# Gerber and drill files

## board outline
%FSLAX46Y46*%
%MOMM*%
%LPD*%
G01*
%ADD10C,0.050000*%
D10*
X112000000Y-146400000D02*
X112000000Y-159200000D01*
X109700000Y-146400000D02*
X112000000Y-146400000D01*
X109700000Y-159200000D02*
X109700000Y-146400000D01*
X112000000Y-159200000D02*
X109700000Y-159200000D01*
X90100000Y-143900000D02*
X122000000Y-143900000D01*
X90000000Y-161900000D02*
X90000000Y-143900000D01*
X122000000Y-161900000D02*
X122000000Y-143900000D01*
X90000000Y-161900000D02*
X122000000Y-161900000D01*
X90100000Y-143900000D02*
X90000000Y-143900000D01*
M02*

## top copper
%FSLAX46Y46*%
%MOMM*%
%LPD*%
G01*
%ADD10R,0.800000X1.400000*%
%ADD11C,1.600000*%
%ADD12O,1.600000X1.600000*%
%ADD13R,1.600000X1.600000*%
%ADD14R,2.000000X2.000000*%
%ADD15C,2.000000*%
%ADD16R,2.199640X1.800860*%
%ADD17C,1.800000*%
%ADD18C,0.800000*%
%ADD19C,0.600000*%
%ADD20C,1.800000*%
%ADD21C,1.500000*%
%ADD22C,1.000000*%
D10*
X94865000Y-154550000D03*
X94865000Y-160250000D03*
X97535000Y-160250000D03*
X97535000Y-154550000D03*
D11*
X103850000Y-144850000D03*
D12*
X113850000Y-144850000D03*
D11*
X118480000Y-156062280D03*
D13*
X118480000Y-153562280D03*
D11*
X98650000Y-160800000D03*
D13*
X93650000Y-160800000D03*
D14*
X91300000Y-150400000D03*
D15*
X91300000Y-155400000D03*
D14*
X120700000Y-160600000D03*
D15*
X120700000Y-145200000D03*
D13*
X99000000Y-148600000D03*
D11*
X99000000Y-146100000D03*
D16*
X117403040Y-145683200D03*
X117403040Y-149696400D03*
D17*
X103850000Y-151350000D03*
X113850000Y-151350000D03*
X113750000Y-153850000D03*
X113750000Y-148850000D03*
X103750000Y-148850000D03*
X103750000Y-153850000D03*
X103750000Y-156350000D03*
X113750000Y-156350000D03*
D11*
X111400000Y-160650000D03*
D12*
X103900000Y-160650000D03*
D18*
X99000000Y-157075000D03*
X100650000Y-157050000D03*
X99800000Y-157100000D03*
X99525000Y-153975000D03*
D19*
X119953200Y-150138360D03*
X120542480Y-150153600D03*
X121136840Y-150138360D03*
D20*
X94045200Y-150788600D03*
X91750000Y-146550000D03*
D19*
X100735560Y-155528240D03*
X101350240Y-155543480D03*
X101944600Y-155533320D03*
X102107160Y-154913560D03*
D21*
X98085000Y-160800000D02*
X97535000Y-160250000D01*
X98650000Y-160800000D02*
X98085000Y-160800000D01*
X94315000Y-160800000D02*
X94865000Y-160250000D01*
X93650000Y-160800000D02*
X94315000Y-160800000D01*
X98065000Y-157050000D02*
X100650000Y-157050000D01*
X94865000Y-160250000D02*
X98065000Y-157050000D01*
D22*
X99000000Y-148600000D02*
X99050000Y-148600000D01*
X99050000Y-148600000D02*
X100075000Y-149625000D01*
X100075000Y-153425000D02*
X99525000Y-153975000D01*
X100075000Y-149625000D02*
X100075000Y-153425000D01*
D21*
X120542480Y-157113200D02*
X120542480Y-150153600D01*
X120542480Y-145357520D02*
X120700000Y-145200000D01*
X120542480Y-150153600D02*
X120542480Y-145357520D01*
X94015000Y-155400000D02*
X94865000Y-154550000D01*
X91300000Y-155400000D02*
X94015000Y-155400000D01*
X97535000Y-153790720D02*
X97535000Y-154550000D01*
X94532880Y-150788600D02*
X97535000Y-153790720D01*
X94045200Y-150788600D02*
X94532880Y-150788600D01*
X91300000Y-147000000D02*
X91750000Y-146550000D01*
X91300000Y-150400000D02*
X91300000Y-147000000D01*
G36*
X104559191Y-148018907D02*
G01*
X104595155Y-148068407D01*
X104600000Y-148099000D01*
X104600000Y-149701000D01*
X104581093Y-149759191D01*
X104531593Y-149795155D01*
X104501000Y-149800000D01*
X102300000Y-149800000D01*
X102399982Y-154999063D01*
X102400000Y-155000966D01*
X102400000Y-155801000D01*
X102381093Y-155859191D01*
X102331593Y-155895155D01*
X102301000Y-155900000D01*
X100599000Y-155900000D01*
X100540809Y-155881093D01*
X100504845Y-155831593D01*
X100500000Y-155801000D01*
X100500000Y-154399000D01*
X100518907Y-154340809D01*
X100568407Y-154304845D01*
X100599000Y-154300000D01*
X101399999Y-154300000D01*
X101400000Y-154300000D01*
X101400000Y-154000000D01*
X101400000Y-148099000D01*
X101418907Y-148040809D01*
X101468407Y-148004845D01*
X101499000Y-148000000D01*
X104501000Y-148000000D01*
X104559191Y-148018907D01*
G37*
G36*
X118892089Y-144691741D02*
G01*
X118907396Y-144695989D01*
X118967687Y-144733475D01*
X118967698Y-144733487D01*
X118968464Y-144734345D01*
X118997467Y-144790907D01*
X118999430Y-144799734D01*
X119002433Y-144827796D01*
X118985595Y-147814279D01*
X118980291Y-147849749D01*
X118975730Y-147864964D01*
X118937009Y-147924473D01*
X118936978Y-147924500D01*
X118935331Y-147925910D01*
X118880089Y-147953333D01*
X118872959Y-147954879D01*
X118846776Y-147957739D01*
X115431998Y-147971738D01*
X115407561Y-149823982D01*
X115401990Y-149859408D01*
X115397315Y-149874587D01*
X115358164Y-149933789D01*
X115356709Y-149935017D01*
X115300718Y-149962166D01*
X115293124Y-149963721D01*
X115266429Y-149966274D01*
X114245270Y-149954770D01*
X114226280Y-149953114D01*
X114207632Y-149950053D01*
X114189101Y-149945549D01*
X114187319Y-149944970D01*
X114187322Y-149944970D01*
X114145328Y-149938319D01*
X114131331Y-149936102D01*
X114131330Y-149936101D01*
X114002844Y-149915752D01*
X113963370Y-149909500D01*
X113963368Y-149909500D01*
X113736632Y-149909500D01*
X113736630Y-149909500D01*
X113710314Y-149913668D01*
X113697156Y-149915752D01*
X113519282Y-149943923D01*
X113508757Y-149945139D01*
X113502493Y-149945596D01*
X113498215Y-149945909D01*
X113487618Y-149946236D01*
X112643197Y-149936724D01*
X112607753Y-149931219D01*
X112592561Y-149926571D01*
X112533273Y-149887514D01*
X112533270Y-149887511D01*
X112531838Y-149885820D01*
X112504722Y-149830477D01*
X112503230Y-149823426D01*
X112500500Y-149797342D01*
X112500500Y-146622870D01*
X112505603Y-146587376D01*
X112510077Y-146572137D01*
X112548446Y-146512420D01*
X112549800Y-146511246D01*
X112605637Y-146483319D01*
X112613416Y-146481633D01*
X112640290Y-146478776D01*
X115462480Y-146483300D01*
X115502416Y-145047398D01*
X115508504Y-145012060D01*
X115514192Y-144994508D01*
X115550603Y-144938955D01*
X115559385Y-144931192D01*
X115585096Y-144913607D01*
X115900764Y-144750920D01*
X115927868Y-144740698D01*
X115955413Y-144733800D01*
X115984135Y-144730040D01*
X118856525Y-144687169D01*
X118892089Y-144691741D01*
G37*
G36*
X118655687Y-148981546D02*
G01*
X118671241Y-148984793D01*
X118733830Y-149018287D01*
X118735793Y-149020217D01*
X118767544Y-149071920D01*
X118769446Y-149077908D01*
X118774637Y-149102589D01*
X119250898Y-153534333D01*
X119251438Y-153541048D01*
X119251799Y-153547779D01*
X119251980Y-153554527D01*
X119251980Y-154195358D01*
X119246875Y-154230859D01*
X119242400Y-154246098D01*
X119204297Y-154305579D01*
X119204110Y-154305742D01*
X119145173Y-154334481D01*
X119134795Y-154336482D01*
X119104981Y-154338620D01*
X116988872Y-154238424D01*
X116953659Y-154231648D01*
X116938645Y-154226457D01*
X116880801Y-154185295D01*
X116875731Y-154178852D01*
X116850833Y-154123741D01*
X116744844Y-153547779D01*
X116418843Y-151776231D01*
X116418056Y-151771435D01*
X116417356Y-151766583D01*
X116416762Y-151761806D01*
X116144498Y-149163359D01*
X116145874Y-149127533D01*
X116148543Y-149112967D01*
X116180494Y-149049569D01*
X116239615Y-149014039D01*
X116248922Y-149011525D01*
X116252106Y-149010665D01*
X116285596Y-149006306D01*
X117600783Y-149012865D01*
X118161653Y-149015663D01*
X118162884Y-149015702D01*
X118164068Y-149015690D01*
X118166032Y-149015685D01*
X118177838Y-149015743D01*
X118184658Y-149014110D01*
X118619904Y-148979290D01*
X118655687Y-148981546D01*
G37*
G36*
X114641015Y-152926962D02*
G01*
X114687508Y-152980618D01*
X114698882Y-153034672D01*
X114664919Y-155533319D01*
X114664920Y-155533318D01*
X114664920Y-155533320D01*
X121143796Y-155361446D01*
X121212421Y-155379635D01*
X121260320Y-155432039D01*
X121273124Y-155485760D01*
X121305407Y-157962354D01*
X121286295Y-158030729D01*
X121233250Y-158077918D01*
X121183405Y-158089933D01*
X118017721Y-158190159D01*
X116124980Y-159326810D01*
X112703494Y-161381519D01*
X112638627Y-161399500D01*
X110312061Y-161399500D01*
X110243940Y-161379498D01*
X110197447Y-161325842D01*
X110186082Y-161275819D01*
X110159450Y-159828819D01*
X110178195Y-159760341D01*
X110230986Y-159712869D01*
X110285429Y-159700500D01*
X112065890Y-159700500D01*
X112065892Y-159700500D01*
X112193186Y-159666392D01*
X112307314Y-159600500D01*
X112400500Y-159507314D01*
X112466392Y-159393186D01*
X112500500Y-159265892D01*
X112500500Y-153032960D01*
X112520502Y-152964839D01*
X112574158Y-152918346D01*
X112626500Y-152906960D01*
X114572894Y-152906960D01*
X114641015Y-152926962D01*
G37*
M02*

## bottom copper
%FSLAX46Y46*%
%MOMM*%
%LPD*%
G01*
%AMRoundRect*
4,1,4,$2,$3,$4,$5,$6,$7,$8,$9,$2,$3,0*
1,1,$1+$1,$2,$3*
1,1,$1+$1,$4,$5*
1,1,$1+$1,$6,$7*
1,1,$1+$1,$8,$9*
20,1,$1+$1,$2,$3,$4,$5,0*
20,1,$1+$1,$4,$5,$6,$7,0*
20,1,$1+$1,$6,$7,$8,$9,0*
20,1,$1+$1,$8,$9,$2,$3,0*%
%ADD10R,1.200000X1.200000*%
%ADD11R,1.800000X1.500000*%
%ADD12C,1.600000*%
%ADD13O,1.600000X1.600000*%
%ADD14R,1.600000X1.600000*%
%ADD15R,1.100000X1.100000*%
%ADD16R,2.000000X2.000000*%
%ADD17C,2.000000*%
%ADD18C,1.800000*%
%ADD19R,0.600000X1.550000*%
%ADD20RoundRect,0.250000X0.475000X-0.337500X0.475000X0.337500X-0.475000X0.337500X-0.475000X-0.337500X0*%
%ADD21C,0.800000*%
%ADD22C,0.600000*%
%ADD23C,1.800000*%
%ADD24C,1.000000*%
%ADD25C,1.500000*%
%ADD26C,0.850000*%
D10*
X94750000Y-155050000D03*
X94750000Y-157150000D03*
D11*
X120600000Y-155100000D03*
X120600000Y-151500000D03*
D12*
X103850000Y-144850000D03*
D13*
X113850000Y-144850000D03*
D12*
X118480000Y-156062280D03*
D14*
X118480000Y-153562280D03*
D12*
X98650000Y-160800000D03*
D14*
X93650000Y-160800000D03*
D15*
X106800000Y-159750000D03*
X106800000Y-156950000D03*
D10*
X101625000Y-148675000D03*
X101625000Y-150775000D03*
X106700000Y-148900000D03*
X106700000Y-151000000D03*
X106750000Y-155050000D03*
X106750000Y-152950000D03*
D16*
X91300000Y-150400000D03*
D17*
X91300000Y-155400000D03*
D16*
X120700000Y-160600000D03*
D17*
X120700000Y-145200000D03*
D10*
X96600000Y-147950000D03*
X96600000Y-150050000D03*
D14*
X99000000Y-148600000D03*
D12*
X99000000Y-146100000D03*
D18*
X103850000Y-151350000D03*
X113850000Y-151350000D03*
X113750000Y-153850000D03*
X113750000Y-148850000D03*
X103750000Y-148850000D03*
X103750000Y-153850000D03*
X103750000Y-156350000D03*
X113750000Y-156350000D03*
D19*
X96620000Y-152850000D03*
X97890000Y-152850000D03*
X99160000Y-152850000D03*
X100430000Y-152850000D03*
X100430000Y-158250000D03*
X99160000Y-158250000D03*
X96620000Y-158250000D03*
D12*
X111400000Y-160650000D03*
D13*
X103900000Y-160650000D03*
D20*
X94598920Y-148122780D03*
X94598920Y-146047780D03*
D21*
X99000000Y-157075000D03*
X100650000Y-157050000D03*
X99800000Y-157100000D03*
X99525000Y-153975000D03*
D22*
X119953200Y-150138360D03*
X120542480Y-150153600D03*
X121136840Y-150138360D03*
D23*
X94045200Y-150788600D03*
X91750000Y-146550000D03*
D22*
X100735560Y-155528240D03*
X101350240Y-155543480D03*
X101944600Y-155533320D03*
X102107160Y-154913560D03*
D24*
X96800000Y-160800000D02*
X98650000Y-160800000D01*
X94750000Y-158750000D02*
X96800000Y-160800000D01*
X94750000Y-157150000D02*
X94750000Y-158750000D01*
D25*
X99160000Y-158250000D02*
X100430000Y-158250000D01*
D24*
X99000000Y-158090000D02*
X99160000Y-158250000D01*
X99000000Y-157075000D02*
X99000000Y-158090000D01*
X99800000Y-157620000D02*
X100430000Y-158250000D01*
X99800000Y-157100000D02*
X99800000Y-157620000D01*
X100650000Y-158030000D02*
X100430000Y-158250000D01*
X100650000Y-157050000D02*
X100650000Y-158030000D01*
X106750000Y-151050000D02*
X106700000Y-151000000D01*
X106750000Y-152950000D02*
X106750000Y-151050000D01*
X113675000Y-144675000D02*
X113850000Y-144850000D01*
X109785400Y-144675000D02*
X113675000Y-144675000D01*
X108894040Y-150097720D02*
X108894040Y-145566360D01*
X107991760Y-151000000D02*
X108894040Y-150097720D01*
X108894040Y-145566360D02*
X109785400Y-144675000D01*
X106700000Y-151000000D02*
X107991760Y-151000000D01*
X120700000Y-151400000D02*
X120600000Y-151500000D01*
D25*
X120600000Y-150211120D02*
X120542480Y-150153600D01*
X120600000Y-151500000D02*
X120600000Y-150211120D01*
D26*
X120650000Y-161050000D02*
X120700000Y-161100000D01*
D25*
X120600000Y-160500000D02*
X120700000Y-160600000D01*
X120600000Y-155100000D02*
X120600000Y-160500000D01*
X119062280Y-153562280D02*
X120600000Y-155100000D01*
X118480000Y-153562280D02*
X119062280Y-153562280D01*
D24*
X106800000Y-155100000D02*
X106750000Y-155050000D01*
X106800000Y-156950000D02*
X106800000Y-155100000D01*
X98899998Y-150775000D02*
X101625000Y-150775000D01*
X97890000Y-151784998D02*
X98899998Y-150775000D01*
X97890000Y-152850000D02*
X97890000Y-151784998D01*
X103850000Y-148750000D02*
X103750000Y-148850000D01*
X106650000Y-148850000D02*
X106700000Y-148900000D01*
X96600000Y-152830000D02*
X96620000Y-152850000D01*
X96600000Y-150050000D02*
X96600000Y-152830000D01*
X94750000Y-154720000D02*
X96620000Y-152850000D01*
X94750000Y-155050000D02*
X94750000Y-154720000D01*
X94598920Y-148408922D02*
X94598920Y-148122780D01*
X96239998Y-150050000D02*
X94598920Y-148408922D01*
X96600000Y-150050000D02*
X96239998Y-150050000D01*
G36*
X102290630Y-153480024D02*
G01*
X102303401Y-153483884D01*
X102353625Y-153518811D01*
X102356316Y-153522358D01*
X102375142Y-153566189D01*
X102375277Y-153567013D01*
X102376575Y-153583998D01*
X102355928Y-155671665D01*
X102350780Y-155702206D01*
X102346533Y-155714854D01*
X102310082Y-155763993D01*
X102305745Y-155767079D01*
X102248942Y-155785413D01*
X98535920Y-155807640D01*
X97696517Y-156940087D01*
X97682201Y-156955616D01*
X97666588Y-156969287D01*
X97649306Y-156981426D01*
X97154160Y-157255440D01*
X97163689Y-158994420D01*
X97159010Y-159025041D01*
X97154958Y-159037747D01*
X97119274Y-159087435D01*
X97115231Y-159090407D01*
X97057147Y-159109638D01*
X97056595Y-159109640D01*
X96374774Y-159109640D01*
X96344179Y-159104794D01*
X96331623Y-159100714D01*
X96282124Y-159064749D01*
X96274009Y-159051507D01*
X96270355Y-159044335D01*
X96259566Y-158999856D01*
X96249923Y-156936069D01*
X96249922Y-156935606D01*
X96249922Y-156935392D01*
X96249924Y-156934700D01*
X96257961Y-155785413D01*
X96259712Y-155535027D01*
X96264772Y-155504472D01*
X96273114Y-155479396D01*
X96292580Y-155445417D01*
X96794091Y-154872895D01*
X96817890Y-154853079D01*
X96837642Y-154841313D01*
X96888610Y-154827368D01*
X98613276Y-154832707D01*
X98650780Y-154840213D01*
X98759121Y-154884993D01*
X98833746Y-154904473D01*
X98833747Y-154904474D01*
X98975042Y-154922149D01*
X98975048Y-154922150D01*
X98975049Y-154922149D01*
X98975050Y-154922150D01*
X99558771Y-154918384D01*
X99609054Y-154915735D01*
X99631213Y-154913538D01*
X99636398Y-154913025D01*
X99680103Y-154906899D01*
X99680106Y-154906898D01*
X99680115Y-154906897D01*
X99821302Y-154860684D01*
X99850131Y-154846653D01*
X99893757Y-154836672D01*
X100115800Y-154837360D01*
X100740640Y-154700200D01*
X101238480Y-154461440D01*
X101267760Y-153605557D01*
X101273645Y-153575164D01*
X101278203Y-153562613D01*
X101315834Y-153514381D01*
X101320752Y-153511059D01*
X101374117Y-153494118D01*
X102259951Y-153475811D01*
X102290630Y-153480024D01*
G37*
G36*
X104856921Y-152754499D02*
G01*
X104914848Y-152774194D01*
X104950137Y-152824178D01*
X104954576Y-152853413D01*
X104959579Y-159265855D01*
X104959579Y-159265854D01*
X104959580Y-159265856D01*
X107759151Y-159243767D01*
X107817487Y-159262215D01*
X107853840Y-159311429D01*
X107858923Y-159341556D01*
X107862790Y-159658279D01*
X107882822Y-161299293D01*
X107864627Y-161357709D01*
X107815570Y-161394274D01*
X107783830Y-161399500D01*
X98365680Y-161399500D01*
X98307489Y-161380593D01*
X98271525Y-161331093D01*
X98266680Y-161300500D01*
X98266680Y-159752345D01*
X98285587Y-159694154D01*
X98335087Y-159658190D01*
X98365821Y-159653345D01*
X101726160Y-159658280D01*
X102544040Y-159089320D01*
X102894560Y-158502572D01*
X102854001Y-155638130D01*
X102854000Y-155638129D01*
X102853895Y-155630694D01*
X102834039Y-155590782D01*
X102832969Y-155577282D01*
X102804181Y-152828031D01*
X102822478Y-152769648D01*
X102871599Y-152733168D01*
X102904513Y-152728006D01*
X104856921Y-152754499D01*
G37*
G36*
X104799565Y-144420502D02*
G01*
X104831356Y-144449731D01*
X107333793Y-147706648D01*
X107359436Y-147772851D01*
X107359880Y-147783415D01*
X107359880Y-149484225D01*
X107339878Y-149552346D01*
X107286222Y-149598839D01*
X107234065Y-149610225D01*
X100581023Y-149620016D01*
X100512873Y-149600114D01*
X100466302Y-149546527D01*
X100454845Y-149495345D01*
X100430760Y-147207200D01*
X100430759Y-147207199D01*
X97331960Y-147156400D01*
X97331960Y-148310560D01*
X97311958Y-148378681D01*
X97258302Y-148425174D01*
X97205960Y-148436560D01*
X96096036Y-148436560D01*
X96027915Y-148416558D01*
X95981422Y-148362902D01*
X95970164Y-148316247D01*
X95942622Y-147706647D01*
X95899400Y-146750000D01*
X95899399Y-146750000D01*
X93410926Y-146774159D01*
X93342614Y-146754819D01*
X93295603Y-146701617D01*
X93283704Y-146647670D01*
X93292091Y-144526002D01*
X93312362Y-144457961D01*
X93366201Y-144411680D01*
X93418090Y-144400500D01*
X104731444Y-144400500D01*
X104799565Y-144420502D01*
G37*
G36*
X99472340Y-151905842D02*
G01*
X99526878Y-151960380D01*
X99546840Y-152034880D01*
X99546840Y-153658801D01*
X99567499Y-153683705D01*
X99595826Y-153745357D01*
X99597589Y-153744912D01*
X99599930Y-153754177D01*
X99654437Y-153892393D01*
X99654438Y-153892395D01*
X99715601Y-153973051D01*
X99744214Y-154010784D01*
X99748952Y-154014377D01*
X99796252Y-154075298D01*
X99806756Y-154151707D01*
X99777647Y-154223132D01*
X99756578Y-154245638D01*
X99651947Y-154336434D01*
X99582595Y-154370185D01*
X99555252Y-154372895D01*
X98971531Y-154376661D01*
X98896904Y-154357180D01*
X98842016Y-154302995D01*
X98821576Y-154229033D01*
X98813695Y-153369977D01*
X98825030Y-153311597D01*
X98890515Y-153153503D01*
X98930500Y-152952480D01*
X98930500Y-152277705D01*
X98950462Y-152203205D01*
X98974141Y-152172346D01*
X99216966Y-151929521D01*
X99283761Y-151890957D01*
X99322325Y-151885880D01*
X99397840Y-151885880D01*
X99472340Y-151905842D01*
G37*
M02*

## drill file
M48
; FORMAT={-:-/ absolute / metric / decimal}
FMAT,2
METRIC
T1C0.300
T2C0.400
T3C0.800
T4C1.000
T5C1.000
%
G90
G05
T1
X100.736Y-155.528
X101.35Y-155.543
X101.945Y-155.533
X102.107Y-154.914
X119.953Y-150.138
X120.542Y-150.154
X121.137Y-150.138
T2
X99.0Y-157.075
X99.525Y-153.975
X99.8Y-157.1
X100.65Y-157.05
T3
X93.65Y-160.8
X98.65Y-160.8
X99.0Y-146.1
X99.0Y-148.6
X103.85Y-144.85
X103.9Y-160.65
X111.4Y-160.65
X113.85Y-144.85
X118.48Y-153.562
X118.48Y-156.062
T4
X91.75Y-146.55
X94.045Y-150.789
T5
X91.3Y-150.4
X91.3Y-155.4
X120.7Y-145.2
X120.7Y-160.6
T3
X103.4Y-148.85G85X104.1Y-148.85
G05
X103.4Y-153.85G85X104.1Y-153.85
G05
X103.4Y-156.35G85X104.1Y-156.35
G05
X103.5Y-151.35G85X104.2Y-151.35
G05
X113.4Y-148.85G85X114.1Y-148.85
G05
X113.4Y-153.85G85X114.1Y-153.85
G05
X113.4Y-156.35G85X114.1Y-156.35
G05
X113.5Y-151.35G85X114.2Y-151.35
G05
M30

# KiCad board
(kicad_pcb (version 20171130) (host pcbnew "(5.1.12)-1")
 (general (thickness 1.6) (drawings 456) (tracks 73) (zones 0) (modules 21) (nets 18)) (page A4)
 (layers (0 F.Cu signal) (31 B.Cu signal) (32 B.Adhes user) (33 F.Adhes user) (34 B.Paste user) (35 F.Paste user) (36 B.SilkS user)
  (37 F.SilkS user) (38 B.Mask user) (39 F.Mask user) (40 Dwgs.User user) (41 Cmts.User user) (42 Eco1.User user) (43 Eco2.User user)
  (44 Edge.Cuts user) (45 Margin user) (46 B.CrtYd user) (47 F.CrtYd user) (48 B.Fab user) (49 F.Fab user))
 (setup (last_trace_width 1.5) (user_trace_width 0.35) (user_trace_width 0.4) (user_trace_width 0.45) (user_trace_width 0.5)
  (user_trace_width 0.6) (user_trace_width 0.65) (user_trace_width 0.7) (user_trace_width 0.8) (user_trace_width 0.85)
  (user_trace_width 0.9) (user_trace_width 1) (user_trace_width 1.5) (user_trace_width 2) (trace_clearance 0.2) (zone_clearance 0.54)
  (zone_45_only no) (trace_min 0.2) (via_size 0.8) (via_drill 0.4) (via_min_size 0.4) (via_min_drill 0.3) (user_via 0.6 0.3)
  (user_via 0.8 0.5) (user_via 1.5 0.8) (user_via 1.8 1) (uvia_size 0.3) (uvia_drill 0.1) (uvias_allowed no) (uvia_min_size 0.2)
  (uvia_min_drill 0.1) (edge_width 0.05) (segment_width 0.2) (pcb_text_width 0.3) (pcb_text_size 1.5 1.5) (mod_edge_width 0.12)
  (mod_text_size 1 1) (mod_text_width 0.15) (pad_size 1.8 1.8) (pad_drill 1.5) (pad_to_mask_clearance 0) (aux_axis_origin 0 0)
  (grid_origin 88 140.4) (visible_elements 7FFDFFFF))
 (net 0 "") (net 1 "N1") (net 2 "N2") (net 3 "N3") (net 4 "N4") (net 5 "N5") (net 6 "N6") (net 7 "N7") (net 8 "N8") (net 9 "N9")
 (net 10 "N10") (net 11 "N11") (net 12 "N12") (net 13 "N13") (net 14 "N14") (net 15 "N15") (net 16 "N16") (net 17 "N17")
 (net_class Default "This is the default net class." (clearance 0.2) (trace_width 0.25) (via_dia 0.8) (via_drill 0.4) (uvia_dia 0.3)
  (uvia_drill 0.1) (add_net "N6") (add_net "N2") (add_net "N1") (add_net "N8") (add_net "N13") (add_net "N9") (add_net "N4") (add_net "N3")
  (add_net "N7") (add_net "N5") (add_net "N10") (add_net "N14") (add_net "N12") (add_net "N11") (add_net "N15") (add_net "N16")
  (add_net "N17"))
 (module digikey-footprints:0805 (layer B.Cu) (at 94.75 156.1 90)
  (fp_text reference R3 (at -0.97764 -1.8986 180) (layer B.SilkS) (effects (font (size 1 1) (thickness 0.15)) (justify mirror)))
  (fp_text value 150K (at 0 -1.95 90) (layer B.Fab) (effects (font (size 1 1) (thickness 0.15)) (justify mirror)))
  (pad 2 smd rect (at 1.05 0 90) (size 1.2 1.2) (layers B.Cu B.Paste B.Mask) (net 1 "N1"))
  (pad 1 smd rect (at -1.05 0 90) (size 1.2 1.2) (layers B.Cu B.Paste B.Mask) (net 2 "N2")))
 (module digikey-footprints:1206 (layer B.Cu) (at 120.6 153.3 90)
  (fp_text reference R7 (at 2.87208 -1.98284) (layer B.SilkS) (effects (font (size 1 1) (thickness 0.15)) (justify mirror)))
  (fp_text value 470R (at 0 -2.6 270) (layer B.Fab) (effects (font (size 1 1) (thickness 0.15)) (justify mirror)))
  (pad 1 smd rect (at -1.8 0 90) (size 1.5 1.8) (layers B.Cu B.Paste B.Mask) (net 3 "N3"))
  (pad 2 smd rect (at 1.8 0 90) (size 1.5 1.8) (layers B.Cu B.Paste B.Mask) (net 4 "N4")))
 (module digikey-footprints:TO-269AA (layer F.Cu) (at 96.2 157.4)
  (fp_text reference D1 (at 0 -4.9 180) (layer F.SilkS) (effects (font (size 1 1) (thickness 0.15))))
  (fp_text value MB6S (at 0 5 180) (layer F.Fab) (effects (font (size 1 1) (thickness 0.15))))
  (pad 4 smd rect (at -1.335 -2.85) (size 0.8 1.4) (layers F.Cu F.Paste F.Mask) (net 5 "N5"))
  (pad 1 smd rect (at -1.335 2.85) (size 0.8 1.4) (layers F.Cu F.Paste F.Mask) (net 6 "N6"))
  (pad 2 smd rect (at 1.335 2.85) (size 0.8 1.4) (layers F.Cu F.Paste F.Mask) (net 2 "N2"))
  (pad 3 smd rect (at 1.335 -2.85) (size 0.8 1.4) (layers F.Cu F.Paste F.Mask) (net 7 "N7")))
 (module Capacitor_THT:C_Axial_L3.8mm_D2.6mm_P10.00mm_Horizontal (layer B.Cu) (at 103.85 144.85)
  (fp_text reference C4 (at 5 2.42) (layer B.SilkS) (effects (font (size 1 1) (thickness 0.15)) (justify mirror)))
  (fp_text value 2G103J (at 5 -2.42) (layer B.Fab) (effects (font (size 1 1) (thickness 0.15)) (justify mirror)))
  (pad 1 thru_hole circle (at 0 0) (size 1.6 1.6) (drill 0.8) (layers *.Cu *.Mask) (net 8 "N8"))
  (pad 2 thru_hole oval (at 10 0) (size 1.6 1.6) (drill 0.8) (layers *.Cu *.Mask) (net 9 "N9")))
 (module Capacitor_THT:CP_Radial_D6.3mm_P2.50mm (layer B.Cu) (at 118.48 153.56228 270)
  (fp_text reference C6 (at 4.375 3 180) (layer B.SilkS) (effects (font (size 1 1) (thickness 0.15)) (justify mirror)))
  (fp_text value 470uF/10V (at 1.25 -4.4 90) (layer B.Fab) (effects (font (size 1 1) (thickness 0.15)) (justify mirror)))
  (pad 2 thru_hole circle (at 2.5 0 270) (size 1.6 1.6) (drill 0.8) (layers *.Cu *.Mask) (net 4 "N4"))
  (pad 1 thru_hole rect (at 0 0 270) (size 1.6 1.6) (drill 0.8) (layers *.Cu *.Mask) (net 3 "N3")))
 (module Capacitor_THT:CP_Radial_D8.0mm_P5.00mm (layer B.Cu) (at 93.65 160.8)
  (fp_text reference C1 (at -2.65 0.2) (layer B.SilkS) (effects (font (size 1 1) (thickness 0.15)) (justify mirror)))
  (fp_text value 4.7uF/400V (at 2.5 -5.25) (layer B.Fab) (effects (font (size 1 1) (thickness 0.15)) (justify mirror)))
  (pad 2 thru_hole circle (at 5 0) (size 1.6 1.6) (drill 0.8) (layers *.Cu *.Mask) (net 2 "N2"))
  (pad 1 thru_hole rect (at 0 0) (size 1.6 1.6) (drill 0.8) (layers *.Cu *.Mask) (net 6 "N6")))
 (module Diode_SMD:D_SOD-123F (layer B.Cu) (at 106.8 158.35 90)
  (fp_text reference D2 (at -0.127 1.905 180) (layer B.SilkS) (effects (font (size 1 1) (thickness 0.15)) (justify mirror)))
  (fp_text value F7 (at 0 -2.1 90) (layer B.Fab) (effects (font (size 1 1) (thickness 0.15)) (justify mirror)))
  (pad 1 smd rect (at -1.4 0 90) (size 1.1 1.1) (layers B.Cu B.Paste B.Mask) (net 2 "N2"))
  (pad 2 smd rect (at 1.4 0 90) (size 1.1 1.1) (layers B.Cu B.Paste B.Mask) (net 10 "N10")))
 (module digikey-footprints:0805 (layer B.Cu) (at 101.625 149.725 270)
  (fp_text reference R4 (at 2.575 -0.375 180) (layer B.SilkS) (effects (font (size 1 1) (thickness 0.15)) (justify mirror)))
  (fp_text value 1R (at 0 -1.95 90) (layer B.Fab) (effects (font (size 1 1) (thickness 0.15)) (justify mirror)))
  (pad 1 smd rect (at -1.05 0 270) (size 1.2 1.2) (layers B.Cu B.Paste B.Mask) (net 8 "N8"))
  (pad 2 smd rect (at 1.05 0 270) (size 1.2 1.2) (layers B.Cu B.Paste B.Mask) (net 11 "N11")))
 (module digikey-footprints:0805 (layer B.Cu) (at 106.7 149.95 90)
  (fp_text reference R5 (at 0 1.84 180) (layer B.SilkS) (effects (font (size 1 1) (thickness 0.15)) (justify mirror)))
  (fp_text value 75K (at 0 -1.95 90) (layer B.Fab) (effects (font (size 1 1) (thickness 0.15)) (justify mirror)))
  (pad 2 smd rect (at 1.05 0 90) (size 1.2 1.2) (layers B.Cu B.Paste B.Mask) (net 8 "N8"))
  (pad 1 smd rect (at -1.05 0 90) (size 1.2 1.2) (layers B.Cu B.Paste B.Mask) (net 9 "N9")))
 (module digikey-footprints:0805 (layer B.Cu) (at 106.75 154 90)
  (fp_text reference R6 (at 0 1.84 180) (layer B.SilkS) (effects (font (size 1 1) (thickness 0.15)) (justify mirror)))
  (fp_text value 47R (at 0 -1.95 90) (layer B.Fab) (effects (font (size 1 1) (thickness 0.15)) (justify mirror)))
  (pad 1 smd rect (at -1.05 0 90) (size 1.2 1.2) (layers B.Cu B.Paste B.Mask) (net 10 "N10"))
  (pad 2 smd rect (at 1.05 0 90) (size 1.2 1.2) (layers B.Cu B.Paste B.Mask) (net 9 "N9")))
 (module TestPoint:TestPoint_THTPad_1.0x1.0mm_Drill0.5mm (layer F.Cu) (at 91.3 150.4)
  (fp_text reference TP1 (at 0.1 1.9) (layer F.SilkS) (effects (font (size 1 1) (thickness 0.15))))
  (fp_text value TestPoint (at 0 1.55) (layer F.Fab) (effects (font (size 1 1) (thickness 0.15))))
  (pad 1 thru_hole rect (at 0 0) (size 2 2) (drill 1) (layers *.Cu *.Mask) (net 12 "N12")))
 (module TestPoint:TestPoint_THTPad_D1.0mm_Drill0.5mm (layer F.Cu) (at 91.3 155.4)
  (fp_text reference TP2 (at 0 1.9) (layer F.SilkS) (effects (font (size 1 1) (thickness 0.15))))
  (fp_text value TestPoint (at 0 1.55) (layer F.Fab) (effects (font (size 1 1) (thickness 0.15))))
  (pad 1 thru_hole circle (at 0 0) (size 2 2) (drill 1) (layers *.Cu *.Mask) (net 5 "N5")))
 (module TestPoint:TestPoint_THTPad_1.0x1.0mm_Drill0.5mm (layer F.Cu) (at 120.7 160.6)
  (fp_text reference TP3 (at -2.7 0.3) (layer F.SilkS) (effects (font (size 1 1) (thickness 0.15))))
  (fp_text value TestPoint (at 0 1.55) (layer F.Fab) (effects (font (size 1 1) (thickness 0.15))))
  (pad 1 thru_hole rect (at 0 0) (size 2 2) (drill 1) (layers *.Cu *.Mask) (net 3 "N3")))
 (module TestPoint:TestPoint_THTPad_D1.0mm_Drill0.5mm (layer F.Cu) (at 120.7 145.2)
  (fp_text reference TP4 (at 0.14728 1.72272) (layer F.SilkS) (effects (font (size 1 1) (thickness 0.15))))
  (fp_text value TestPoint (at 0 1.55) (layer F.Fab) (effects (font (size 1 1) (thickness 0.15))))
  (pad 1 thru_hole circle (at 0 0) (size 2 2) (drill 1) (layers *.Cu *.Mask) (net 4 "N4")))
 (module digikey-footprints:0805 (layer B.Cu) (at 96.6 149 90)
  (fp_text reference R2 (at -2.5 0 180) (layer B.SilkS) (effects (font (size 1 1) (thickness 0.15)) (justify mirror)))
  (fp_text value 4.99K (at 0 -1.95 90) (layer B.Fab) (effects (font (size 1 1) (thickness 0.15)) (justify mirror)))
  (pad 2 smd rect (at 1.05 0 90) (size 1.2 1.2) (layers B.Cu B.Paste B.Mask) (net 8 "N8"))
  (pad 1 smd rect (at -1.05 0 90) (size 1.2 1.2) (layers B.Cu B.Paste B.Mask) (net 1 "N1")))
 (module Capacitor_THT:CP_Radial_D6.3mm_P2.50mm (layer F.Cu) (at 99 148.6 90)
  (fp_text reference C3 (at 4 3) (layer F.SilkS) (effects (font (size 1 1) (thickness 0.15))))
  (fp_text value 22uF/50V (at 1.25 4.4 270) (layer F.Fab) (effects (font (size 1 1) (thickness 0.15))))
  (pad 1 thru_hole rect (at 0 0 90) (size 1.6 1.6) (drill 0.8) (layers *.Cu *.Mask) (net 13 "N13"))
  (pad 2 thru_hole circle (at 2.5 0 90) (size 1.6 1.6) (drill 0.8) (layers *.Cu *.Mask) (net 8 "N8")))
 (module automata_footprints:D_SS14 (layer F.Cu) (at 117.40304 147.6898 90)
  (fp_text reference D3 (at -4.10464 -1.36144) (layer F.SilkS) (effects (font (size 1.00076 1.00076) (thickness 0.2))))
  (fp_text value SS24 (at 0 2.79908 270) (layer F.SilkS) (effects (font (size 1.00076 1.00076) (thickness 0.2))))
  (pad 2 smd rect (at 2.0066 0 90) (size 1.80086 2.19964) (layers F.Cu F.Paste F.Mask) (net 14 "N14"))
  (pad 1 smd rect (at -2.0066 0 90) (size 1.80086 2.19964) (layers F.Cu F.Paste F.Mask) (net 3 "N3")))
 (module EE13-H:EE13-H (layer F.Cu) (at 108.75 151.35)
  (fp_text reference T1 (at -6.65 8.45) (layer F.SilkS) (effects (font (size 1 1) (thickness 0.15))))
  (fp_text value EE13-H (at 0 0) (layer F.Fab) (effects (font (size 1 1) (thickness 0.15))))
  (pad 2 thru_hole circle (at -4.9 0) (size 1.8 1.8) (drill oval 1.5 0.8) (layers *.Cu *.Mask) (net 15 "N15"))
  (pad 7 thru_hole circle (at 5.1 0) (size 1.8 1.8) (drill oval 1.5 0.8) (layers *.Cu *.Mask) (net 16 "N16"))
  (pad 6 thru_hole circle (at 5 2.5) (size 1.8 1.8) (drill oval 1.5 0.8) (layers *.Cu *.Mask) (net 4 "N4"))
  (pad 8 thru_hole circle (at 5 -2.5) (size 1.8 1.8) (drill oval 1.5 0.8) (layers *.Cu *.Mask) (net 14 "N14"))
  (pad 1 thru_hole circle (at -5 -2.5) (size 1.8 1.8) (drill oval 1.5 0.8) (layers *.Cu *.Mask) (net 8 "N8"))
  (pad 3 thru_hole circle (at -5 2.5) (size 1.8 1.8) (drill oval 1.5 0.8) (layers *.Cu *.Mask) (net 2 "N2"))
  (pad 4 thru_hole circle (at -5 5) (size 1.8 1.8) (drill oval 1.5 0.8) (layers *.Cu *.Mask) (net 2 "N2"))
  (pad 5 thru_hole circle (at 5 5) (size 1.8 1.8) (drill oval 1.5 0.8) (layers *.Cu *.Mask) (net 4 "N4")))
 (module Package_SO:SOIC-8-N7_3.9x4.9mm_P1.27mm (layer B.Cu) (at 98.525 155.55 270)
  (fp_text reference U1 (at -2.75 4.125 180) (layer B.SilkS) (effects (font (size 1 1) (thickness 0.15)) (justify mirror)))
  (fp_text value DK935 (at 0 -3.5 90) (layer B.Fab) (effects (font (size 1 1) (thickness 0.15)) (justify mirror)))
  (pad 1 smd rect (at -2.7 1.905 270) (size 1.55 0.6) (layers B.Cu B.Paste B.Mask) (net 1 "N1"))
  (pad 2 smd rect (at -2.7 0.635 270) (size 1.55 0.6) (layers B.Cu B.Paste B.Mask) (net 11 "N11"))
  (pad 3 smd rect (at -2.7 -0.635 270) (size 1.55 0.6) (layers B.Cu B.Paste B.Mask) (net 13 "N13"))
  (pad 4 smd rect (at -2.7 -1.905 270) (size 1.55 0.6) (layers B.Cu B.Paste B.Mask) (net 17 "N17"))
  (pad 5 smd rect (at 2.7 -1.905 270) (size 1.55 0.6) (layers B.Cu B.Paste B.Mask) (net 6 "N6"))
  (pad 6 smd rect (at 2.7 -0.635 270) (size 1.55 0.6) (layers B.Cu B.Paste B.Mask) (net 6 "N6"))
  (pad 8 smd rect (at 2.7 1.905 270) (size 1.55 0.6) (layers B.Cu B.Paste B.Mask) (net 8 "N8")))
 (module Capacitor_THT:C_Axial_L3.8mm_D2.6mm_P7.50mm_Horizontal (layer F.Cu) (at 111.4 160.65 180)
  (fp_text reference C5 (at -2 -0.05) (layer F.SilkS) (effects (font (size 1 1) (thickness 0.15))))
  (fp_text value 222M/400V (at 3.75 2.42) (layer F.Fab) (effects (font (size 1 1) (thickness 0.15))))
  (pad 1 thru_hole circle (at 0 0 180) (size 1.6 1.6) (drill 0.8) (layers *.Cu *.Mask) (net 4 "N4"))
  (pad 2 thru_hole oval (at 7.5 0 180) (size 1.6 1.6) (drill 0.8) (layers *.Cu *.Mask) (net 2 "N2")))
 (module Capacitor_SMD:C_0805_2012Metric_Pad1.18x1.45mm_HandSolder (layer B.Cu) (at 94.59892 147.08528 90)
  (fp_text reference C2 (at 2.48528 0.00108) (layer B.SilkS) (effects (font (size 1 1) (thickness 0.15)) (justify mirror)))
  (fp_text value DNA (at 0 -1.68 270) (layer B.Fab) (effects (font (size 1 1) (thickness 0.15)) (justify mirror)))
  (pad 1 smd roundrect (at -1.0375 0 90) (size 1.175 1.45) (layers B.Cu B.Paste B.Mask) (roundrect_rratio 0.212766) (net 1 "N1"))
  (pad 2 smd roundrect (at 1.0375 0 90) (size 1.175 1.45) (layers B.Cu B.Paste B.Mask) (roundrect_rratio 0.212766) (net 8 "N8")))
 (gr_line (start 112 146.4) (end 112 159.2) (layer Edge.Cuts) (width 0.05))
 (gr_line (start 109.7 146.4) (end 112 146.4) (layer Edge.Cuts) (width 0.05))
 (gr_line (start 109.7 159.2) (end 109.7 146.4) (layer Edge.Cuts) (width 0.05))
 (gr_line (start 112 159.2) (end 109.7 159.2) (layer Edge.Cuts) (width 0.05))
 (gr_line (start 90.1 143.9) (end 122 143.9) (layer Edge.Cuts) (width 0.05))
 (gr_line (start 90 161.9) (end 90 143.9) (layer Edge.Cuts) (width 0.05))
 (gr_line (start 122 161.9) (end 122 143.9) (layer Edge.Cuts) (width 0.05))
 (gr_line (start 90 161.9) (end 122 161.9) (layer Edge.Cuts) (width 0.05))
 (gr_line (start 90.1 143.9) (end 90 143.9) (layer Edge.Cuts) (width 0.05))
 (segment (start 98.085 160.8) (end 97.535 160.25) (width 1.5) (layer F.Cu) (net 2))
 (segment (start 98.65 160.8) (end 98.085 160.8) (width 1.5) (layer F.Cu) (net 2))
 (segment (start 96.8 160.8) (end 98.65 160.8) (width 1) (layer B.Cu) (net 2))
 (segment (start 94.75 158.75) (end 96.8 160.8) (width 1) (layer B.Cu) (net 2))
 (segment (start 94.75 157.15) (end 94.75 158.75) (width 1) (layer B.Cu) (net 2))
 (via (at 99 157.075) (size 0.8) (drill 0.4) (layers F.Cu B.Cu) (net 6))
 (via (at 100.65 157.05) (size 0.8) (drill 0.4) (layers F.Cu B.Cu) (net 6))
 (via (at 99.8 157.1) (size 0.8) (drill 0.4) (layers F.Cu B.Cu) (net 6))
 (segment (start 94.315 160.8) (end 94.865 160.25) (width 1.5) (layer F.Cu) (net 6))
 (segment (start 93.65 160.8) (end 94.315 160.8) (width 1.5) (layer F.Cu) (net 6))
 (segment (start 98.065 157.05) (end 100.65 157.05) (width 1.5) (layer F.Cu) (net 6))
 (segment (start 94.865 160.25) (end 98.065 157.05) (width 1.5) (layer F.Cu) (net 6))
 (segment (start 99.16 158.25) (end 100.43 158.25) (width 1.5) (layer B.Cu) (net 6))
 (segment (start 99 158.09) (end 99.16 158.25) (width 1) (layer B.Cu) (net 6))
 (segment (start 99 157.075) (end 99 158.09) (width 1) (layer B.Cu) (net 6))
 (segment (start 99.8 157.62) (end 100.43 158.25) (width 1) (layer B.Cu) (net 6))
 (segment (start 99.8 157.1) (end 99.8 157.62) (width 1) (layer B.Cu) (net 6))
 (segment (start 100.65 158.03) (end 100.43 158.25) (width 1) (layer B.Cu) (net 6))
 (segment (start 100.65 157.05) (end 100.65 158.03) (width 1) (layer B.Cu) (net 6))
 (segment (start 99 148.6) (end 99.05 148.6) (width 1) (layer F.Cu) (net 13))
 (segment (start 99.05 148.6) (end 100.075 149.625) (width 1) (layer F.Cu) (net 13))
 (segment (start 100.075 153.425) (end 99.525 153.975) (width 1) (layer F.Cu) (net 13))
 (segment (start 100.075 149.625) (end 100.075 153.425) (width 1) (layer F.Cu) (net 13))
 (via (at 99.525 153.975) (size 0.8) (drill 0.4) (layers F.Cu B.Cu) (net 13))
 (segment (start 106.75 151.05) (end 106.7 151) (width 1) (layer B.Cu) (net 9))
 (segment (start 106.75 152.95) (end 106.75 151.05) (width 1) (layer B.Cu) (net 9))
 (segment (start 113.675 144.675) (end 113.85 144.85) (width 1) (layer B.Cu) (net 9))
 (segment (start 109.7854 144.675) (end 113.675 144.675) (width 1) (layer B.Cu) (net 9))
 (segment (start 108.89404 150.09772) (end 108.89404 145.56636) (width 1) (layer B.Cu) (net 9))
 (segment (start 107.99176 151) (end 108.89404 150.09772) (width 1) (layer B.Cu) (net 9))
 (segment (start 108.89404 145.56636) (end 109.7854 144.675) (width 1) (layer B.Cu) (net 9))
 (segment (start 106.7 151) (end 107.99176 151) (width 1) (layer B.Cu) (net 9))
 (via (at 119.9532 150.13836) (size 0.6) (drill 0.3) (layers F.Cu B.Cu) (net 4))
 (via (at 120.54248 150.1536) (size 0.6) (drill 0.3) (layers F.Cu B.Cu) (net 4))
 (via (at 121.13684 150.13836) (size 0.6) (drill 0.3) (layers F.Cu B.Cu) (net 4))
 (segment (start 120.7 151.4) (end 120.6 151.5) (width 1) (layer B.Cu) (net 4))
 (segment (start 120.6 150.21112) (end 120.54248 150.1536) (width 1.5) (layer B.Cu) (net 4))
 (segment (start 120.6 151.5) (end 120.6 150.21112) (width 1.5) (layer B.Cu) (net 4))
 (segment (start 120.54248 157.1132) (end 120.54248 150.1536) (width 1.5) (layer F.Cu) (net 4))
 (segment (start 120.54248 145.35752) (end 120.7 145.2) (width 1.5) (layer F.Cu) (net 4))
 (segment (start 120.54248 150.1536) (end 120.54248 145.35752) (width 1.5) (layer F.Cu) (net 4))
 (segment (start 120.65 161.05) (end 120.7 161.1) (width 0.85) (layer B.Cu) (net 3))
 (segment (start 120.6 160.5) (end 120.7 160.6) (width 1.5) (layer B.Cu) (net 3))
 (segment (start 120.6 155.1) (end 120.6 160.5) (width 1.5) (layer B.Cu) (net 3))
 (segment (start 119.06228 153.56228) (end 120.6 155.1) (width 1.5) (layer B.Cu) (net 3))
 (segment (start 118.48 153.56228) (end 119.06228 153.56228) (width 1.5) (layer B.Cu) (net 3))
 (segment (start 94.015 155.4) (end 94.865 154.55) (width 1.5) (layer F.Cu) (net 5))
 (segment (start 91.3 155.4) (end 94.015 155.4) (width 1.5) (layer F.Cu) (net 5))
 (via (at 94.0452 150.7886) (size 1.8) (drill 1) (layers F.Cu B.Cu) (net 7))
 (segment (start 97.535 153.79072) (end 97.535 154.55) (width 1.5) (layer F.Cu) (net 7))
 (segment (start 94.53288 150.7886) (end 97.535 153.79072) (width 1.5) (layer F.Cu) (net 7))
 (segment (start 94.0452 150.7886) (end 94.53288 150.7886) (width 1.5) (layer F.Cu) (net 7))
 (segment (start 106.8 155.1) (end 106.75 155.05) (width 1) (layer B.Cu) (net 10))
 (segment (start 106.8 156.95) (end 106.8 155.1) (width 1) (layer B.Cu) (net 10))
 (via (at 91.75 146.55) (size 1.8) (drill 1) (layers F.Cu B.Cu) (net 12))
 (segment (start 91.3 147) (end 91.75 146.55) (width 1.5) (layer F.Cu) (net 12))
 (segment (start 91.3 150.4) (end 91.3 147) (width 1.5) (layer F.Cu) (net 12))
 (segment (start 98.899998 150.775) (end 101.625 150.775) (width 1) (layer B.Cu) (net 11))
 (segment (start 97.89 151.784998) (end 98.899998 150.775) (width 1) (layer B.Cu) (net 11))
 (segment (start 97.89 152.85) (end 97.89 151.784998) (width 1) (layer B.Cu) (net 11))
 (segment (start 103.85 148.75) (end 103.75 148.85) (width 1) (layer B.Cu) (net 8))
 (segment (start 106.65 148.85) (end 106.7 148.9) (width 1) (layer B.Cu) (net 8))
 (via (at 100.73556 155.52824) (size 0.6) (drill 0.3) (layers F.Cu B.Cu) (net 8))
 (via (at 101.35024 155.54348) (size 0.6) (drill 0.3) (layers F.Cu B.Cu) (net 8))
 (via (at 101.9446 155.53332) (size 0.6) (drill 0.3) (layers F.Cu B.Cu) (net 8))
 (via (at 102.10716 154.91356) (size 0.6) (drill 0.3) (layers F.Cu B.Cu) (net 8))
 (segment (start 96.6 152.83) (end 96.62 152.85) (width 1) (layer B.Cu) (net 1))
 (segment (start 96.6 150.05) (end 96.6 152.83) (width 1) (layer B.Cu) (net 1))
 (segment (start 94.75 154.72) (end 96.62 152.85) (width 1) (layer B.Cu) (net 1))
 (segment (start 94.75 155.05) (end 94.75 154.72) (width 1) (layer B.Cu) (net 1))
 (segment (start 94.59892 148.408922) (end 94.59892 148.12278) (width 1) (layer B.Cu) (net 1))
 (segment (start 96.239998 150.05) (end 94.59892 148.408922) (width 1) (layer B.Cu) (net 1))
 (segment (start 96.6 150.05) (end 96.239998 150.05) (width 1) (layer B.Cu) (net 1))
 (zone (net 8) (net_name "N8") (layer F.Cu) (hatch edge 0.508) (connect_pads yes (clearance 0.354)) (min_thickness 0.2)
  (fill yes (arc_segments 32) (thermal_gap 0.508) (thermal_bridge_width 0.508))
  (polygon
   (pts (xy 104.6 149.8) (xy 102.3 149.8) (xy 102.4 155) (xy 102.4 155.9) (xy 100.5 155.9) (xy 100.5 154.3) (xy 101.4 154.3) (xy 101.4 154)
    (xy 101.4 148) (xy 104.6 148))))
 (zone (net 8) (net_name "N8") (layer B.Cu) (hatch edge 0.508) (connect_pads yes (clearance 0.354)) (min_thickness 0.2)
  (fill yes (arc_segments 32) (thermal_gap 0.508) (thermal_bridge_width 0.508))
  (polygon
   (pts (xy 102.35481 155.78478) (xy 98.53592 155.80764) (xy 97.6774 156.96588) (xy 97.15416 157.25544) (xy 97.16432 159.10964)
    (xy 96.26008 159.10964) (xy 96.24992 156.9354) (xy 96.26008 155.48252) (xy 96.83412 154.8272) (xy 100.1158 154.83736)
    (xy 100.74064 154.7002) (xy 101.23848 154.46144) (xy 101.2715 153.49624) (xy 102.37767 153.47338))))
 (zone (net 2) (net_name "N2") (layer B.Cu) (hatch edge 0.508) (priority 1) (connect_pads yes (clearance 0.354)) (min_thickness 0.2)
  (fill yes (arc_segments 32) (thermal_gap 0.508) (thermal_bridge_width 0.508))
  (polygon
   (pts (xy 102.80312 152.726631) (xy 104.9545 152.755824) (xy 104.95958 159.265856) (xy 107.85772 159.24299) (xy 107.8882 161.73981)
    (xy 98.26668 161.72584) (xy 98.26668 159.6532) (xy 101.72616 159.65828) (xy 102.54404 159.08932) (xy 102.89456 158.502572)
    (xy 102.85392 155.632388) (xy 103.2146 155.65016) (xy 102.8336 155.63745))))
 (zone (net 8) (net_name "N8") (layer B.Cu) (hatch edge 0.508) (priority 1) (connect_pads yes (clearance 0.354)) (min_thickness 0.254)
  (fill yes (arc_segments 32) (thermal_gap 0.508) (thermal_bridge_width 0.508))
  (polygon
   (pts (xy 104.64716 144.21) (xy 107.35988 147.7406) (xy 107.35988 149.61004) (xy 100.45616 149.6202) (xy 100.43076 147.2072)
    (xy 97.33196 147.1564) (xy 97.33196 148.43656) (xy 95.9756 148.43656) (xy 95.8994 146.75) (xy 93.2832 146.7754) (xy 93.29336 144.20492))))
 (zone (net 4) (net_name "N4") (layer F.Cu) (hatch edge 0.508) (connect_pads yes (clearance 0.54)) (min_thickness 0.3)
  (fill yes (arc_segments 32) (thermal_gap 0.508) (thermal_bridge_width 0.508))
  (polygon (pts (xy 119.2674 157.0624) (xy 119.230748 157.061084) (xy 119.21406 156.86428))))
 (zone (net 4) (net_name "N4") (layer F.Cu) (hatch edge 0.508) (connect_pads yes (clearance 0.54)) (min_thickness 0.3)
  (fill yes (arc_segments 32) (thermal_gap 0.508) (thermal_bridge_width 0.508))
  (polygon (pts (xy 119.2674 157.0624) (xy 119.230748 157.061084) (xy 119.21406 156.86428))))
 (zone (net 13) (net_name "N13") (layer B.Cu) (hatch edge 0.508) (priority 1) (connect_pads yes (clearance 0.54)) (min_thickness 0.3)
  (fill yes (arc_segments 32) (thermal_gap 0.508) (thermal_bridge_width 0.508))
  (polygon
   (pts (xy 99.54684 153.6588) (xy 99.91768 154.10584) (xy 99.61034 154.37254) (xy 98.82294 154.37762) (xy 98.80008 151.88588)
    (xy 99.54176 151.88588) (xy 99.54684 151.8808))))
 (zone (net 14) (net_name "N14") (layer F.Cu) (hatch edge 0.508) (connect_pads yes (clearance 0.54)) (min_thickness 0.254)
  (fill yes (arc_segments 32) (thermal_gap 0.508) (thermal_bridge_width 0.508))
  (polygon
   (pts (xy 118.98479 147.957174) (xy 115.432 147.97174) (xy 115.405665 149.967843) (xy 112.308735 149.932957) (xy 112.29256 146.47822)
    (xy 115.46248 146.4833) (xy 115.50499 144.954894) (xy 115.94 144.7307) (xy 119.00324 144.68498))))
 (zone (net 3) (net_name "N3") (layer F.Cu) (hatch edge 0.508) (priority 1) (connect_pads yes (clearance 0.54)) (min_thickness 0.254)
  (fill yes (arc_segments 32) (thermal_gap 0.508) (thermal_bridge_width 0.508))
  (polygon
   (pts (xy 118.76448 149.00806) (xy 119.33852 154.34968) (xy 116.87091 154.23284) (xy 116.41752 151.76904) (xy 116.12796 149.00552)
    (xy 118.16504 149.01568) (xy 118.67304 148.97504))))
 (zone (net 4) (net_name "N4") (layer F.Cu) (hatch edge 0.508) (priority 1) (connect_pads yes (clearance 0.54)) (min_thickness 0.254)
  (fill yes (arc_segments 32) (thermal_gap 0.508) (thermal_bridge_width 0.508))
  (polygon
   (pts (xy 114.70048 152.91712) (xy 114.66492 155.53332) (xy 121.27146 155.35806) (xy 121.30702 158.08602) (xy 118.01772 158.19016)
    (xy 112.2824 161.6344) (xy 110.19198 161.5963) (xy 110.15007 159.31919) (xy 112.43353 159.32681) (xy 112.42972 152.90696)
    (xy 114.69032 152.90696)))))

